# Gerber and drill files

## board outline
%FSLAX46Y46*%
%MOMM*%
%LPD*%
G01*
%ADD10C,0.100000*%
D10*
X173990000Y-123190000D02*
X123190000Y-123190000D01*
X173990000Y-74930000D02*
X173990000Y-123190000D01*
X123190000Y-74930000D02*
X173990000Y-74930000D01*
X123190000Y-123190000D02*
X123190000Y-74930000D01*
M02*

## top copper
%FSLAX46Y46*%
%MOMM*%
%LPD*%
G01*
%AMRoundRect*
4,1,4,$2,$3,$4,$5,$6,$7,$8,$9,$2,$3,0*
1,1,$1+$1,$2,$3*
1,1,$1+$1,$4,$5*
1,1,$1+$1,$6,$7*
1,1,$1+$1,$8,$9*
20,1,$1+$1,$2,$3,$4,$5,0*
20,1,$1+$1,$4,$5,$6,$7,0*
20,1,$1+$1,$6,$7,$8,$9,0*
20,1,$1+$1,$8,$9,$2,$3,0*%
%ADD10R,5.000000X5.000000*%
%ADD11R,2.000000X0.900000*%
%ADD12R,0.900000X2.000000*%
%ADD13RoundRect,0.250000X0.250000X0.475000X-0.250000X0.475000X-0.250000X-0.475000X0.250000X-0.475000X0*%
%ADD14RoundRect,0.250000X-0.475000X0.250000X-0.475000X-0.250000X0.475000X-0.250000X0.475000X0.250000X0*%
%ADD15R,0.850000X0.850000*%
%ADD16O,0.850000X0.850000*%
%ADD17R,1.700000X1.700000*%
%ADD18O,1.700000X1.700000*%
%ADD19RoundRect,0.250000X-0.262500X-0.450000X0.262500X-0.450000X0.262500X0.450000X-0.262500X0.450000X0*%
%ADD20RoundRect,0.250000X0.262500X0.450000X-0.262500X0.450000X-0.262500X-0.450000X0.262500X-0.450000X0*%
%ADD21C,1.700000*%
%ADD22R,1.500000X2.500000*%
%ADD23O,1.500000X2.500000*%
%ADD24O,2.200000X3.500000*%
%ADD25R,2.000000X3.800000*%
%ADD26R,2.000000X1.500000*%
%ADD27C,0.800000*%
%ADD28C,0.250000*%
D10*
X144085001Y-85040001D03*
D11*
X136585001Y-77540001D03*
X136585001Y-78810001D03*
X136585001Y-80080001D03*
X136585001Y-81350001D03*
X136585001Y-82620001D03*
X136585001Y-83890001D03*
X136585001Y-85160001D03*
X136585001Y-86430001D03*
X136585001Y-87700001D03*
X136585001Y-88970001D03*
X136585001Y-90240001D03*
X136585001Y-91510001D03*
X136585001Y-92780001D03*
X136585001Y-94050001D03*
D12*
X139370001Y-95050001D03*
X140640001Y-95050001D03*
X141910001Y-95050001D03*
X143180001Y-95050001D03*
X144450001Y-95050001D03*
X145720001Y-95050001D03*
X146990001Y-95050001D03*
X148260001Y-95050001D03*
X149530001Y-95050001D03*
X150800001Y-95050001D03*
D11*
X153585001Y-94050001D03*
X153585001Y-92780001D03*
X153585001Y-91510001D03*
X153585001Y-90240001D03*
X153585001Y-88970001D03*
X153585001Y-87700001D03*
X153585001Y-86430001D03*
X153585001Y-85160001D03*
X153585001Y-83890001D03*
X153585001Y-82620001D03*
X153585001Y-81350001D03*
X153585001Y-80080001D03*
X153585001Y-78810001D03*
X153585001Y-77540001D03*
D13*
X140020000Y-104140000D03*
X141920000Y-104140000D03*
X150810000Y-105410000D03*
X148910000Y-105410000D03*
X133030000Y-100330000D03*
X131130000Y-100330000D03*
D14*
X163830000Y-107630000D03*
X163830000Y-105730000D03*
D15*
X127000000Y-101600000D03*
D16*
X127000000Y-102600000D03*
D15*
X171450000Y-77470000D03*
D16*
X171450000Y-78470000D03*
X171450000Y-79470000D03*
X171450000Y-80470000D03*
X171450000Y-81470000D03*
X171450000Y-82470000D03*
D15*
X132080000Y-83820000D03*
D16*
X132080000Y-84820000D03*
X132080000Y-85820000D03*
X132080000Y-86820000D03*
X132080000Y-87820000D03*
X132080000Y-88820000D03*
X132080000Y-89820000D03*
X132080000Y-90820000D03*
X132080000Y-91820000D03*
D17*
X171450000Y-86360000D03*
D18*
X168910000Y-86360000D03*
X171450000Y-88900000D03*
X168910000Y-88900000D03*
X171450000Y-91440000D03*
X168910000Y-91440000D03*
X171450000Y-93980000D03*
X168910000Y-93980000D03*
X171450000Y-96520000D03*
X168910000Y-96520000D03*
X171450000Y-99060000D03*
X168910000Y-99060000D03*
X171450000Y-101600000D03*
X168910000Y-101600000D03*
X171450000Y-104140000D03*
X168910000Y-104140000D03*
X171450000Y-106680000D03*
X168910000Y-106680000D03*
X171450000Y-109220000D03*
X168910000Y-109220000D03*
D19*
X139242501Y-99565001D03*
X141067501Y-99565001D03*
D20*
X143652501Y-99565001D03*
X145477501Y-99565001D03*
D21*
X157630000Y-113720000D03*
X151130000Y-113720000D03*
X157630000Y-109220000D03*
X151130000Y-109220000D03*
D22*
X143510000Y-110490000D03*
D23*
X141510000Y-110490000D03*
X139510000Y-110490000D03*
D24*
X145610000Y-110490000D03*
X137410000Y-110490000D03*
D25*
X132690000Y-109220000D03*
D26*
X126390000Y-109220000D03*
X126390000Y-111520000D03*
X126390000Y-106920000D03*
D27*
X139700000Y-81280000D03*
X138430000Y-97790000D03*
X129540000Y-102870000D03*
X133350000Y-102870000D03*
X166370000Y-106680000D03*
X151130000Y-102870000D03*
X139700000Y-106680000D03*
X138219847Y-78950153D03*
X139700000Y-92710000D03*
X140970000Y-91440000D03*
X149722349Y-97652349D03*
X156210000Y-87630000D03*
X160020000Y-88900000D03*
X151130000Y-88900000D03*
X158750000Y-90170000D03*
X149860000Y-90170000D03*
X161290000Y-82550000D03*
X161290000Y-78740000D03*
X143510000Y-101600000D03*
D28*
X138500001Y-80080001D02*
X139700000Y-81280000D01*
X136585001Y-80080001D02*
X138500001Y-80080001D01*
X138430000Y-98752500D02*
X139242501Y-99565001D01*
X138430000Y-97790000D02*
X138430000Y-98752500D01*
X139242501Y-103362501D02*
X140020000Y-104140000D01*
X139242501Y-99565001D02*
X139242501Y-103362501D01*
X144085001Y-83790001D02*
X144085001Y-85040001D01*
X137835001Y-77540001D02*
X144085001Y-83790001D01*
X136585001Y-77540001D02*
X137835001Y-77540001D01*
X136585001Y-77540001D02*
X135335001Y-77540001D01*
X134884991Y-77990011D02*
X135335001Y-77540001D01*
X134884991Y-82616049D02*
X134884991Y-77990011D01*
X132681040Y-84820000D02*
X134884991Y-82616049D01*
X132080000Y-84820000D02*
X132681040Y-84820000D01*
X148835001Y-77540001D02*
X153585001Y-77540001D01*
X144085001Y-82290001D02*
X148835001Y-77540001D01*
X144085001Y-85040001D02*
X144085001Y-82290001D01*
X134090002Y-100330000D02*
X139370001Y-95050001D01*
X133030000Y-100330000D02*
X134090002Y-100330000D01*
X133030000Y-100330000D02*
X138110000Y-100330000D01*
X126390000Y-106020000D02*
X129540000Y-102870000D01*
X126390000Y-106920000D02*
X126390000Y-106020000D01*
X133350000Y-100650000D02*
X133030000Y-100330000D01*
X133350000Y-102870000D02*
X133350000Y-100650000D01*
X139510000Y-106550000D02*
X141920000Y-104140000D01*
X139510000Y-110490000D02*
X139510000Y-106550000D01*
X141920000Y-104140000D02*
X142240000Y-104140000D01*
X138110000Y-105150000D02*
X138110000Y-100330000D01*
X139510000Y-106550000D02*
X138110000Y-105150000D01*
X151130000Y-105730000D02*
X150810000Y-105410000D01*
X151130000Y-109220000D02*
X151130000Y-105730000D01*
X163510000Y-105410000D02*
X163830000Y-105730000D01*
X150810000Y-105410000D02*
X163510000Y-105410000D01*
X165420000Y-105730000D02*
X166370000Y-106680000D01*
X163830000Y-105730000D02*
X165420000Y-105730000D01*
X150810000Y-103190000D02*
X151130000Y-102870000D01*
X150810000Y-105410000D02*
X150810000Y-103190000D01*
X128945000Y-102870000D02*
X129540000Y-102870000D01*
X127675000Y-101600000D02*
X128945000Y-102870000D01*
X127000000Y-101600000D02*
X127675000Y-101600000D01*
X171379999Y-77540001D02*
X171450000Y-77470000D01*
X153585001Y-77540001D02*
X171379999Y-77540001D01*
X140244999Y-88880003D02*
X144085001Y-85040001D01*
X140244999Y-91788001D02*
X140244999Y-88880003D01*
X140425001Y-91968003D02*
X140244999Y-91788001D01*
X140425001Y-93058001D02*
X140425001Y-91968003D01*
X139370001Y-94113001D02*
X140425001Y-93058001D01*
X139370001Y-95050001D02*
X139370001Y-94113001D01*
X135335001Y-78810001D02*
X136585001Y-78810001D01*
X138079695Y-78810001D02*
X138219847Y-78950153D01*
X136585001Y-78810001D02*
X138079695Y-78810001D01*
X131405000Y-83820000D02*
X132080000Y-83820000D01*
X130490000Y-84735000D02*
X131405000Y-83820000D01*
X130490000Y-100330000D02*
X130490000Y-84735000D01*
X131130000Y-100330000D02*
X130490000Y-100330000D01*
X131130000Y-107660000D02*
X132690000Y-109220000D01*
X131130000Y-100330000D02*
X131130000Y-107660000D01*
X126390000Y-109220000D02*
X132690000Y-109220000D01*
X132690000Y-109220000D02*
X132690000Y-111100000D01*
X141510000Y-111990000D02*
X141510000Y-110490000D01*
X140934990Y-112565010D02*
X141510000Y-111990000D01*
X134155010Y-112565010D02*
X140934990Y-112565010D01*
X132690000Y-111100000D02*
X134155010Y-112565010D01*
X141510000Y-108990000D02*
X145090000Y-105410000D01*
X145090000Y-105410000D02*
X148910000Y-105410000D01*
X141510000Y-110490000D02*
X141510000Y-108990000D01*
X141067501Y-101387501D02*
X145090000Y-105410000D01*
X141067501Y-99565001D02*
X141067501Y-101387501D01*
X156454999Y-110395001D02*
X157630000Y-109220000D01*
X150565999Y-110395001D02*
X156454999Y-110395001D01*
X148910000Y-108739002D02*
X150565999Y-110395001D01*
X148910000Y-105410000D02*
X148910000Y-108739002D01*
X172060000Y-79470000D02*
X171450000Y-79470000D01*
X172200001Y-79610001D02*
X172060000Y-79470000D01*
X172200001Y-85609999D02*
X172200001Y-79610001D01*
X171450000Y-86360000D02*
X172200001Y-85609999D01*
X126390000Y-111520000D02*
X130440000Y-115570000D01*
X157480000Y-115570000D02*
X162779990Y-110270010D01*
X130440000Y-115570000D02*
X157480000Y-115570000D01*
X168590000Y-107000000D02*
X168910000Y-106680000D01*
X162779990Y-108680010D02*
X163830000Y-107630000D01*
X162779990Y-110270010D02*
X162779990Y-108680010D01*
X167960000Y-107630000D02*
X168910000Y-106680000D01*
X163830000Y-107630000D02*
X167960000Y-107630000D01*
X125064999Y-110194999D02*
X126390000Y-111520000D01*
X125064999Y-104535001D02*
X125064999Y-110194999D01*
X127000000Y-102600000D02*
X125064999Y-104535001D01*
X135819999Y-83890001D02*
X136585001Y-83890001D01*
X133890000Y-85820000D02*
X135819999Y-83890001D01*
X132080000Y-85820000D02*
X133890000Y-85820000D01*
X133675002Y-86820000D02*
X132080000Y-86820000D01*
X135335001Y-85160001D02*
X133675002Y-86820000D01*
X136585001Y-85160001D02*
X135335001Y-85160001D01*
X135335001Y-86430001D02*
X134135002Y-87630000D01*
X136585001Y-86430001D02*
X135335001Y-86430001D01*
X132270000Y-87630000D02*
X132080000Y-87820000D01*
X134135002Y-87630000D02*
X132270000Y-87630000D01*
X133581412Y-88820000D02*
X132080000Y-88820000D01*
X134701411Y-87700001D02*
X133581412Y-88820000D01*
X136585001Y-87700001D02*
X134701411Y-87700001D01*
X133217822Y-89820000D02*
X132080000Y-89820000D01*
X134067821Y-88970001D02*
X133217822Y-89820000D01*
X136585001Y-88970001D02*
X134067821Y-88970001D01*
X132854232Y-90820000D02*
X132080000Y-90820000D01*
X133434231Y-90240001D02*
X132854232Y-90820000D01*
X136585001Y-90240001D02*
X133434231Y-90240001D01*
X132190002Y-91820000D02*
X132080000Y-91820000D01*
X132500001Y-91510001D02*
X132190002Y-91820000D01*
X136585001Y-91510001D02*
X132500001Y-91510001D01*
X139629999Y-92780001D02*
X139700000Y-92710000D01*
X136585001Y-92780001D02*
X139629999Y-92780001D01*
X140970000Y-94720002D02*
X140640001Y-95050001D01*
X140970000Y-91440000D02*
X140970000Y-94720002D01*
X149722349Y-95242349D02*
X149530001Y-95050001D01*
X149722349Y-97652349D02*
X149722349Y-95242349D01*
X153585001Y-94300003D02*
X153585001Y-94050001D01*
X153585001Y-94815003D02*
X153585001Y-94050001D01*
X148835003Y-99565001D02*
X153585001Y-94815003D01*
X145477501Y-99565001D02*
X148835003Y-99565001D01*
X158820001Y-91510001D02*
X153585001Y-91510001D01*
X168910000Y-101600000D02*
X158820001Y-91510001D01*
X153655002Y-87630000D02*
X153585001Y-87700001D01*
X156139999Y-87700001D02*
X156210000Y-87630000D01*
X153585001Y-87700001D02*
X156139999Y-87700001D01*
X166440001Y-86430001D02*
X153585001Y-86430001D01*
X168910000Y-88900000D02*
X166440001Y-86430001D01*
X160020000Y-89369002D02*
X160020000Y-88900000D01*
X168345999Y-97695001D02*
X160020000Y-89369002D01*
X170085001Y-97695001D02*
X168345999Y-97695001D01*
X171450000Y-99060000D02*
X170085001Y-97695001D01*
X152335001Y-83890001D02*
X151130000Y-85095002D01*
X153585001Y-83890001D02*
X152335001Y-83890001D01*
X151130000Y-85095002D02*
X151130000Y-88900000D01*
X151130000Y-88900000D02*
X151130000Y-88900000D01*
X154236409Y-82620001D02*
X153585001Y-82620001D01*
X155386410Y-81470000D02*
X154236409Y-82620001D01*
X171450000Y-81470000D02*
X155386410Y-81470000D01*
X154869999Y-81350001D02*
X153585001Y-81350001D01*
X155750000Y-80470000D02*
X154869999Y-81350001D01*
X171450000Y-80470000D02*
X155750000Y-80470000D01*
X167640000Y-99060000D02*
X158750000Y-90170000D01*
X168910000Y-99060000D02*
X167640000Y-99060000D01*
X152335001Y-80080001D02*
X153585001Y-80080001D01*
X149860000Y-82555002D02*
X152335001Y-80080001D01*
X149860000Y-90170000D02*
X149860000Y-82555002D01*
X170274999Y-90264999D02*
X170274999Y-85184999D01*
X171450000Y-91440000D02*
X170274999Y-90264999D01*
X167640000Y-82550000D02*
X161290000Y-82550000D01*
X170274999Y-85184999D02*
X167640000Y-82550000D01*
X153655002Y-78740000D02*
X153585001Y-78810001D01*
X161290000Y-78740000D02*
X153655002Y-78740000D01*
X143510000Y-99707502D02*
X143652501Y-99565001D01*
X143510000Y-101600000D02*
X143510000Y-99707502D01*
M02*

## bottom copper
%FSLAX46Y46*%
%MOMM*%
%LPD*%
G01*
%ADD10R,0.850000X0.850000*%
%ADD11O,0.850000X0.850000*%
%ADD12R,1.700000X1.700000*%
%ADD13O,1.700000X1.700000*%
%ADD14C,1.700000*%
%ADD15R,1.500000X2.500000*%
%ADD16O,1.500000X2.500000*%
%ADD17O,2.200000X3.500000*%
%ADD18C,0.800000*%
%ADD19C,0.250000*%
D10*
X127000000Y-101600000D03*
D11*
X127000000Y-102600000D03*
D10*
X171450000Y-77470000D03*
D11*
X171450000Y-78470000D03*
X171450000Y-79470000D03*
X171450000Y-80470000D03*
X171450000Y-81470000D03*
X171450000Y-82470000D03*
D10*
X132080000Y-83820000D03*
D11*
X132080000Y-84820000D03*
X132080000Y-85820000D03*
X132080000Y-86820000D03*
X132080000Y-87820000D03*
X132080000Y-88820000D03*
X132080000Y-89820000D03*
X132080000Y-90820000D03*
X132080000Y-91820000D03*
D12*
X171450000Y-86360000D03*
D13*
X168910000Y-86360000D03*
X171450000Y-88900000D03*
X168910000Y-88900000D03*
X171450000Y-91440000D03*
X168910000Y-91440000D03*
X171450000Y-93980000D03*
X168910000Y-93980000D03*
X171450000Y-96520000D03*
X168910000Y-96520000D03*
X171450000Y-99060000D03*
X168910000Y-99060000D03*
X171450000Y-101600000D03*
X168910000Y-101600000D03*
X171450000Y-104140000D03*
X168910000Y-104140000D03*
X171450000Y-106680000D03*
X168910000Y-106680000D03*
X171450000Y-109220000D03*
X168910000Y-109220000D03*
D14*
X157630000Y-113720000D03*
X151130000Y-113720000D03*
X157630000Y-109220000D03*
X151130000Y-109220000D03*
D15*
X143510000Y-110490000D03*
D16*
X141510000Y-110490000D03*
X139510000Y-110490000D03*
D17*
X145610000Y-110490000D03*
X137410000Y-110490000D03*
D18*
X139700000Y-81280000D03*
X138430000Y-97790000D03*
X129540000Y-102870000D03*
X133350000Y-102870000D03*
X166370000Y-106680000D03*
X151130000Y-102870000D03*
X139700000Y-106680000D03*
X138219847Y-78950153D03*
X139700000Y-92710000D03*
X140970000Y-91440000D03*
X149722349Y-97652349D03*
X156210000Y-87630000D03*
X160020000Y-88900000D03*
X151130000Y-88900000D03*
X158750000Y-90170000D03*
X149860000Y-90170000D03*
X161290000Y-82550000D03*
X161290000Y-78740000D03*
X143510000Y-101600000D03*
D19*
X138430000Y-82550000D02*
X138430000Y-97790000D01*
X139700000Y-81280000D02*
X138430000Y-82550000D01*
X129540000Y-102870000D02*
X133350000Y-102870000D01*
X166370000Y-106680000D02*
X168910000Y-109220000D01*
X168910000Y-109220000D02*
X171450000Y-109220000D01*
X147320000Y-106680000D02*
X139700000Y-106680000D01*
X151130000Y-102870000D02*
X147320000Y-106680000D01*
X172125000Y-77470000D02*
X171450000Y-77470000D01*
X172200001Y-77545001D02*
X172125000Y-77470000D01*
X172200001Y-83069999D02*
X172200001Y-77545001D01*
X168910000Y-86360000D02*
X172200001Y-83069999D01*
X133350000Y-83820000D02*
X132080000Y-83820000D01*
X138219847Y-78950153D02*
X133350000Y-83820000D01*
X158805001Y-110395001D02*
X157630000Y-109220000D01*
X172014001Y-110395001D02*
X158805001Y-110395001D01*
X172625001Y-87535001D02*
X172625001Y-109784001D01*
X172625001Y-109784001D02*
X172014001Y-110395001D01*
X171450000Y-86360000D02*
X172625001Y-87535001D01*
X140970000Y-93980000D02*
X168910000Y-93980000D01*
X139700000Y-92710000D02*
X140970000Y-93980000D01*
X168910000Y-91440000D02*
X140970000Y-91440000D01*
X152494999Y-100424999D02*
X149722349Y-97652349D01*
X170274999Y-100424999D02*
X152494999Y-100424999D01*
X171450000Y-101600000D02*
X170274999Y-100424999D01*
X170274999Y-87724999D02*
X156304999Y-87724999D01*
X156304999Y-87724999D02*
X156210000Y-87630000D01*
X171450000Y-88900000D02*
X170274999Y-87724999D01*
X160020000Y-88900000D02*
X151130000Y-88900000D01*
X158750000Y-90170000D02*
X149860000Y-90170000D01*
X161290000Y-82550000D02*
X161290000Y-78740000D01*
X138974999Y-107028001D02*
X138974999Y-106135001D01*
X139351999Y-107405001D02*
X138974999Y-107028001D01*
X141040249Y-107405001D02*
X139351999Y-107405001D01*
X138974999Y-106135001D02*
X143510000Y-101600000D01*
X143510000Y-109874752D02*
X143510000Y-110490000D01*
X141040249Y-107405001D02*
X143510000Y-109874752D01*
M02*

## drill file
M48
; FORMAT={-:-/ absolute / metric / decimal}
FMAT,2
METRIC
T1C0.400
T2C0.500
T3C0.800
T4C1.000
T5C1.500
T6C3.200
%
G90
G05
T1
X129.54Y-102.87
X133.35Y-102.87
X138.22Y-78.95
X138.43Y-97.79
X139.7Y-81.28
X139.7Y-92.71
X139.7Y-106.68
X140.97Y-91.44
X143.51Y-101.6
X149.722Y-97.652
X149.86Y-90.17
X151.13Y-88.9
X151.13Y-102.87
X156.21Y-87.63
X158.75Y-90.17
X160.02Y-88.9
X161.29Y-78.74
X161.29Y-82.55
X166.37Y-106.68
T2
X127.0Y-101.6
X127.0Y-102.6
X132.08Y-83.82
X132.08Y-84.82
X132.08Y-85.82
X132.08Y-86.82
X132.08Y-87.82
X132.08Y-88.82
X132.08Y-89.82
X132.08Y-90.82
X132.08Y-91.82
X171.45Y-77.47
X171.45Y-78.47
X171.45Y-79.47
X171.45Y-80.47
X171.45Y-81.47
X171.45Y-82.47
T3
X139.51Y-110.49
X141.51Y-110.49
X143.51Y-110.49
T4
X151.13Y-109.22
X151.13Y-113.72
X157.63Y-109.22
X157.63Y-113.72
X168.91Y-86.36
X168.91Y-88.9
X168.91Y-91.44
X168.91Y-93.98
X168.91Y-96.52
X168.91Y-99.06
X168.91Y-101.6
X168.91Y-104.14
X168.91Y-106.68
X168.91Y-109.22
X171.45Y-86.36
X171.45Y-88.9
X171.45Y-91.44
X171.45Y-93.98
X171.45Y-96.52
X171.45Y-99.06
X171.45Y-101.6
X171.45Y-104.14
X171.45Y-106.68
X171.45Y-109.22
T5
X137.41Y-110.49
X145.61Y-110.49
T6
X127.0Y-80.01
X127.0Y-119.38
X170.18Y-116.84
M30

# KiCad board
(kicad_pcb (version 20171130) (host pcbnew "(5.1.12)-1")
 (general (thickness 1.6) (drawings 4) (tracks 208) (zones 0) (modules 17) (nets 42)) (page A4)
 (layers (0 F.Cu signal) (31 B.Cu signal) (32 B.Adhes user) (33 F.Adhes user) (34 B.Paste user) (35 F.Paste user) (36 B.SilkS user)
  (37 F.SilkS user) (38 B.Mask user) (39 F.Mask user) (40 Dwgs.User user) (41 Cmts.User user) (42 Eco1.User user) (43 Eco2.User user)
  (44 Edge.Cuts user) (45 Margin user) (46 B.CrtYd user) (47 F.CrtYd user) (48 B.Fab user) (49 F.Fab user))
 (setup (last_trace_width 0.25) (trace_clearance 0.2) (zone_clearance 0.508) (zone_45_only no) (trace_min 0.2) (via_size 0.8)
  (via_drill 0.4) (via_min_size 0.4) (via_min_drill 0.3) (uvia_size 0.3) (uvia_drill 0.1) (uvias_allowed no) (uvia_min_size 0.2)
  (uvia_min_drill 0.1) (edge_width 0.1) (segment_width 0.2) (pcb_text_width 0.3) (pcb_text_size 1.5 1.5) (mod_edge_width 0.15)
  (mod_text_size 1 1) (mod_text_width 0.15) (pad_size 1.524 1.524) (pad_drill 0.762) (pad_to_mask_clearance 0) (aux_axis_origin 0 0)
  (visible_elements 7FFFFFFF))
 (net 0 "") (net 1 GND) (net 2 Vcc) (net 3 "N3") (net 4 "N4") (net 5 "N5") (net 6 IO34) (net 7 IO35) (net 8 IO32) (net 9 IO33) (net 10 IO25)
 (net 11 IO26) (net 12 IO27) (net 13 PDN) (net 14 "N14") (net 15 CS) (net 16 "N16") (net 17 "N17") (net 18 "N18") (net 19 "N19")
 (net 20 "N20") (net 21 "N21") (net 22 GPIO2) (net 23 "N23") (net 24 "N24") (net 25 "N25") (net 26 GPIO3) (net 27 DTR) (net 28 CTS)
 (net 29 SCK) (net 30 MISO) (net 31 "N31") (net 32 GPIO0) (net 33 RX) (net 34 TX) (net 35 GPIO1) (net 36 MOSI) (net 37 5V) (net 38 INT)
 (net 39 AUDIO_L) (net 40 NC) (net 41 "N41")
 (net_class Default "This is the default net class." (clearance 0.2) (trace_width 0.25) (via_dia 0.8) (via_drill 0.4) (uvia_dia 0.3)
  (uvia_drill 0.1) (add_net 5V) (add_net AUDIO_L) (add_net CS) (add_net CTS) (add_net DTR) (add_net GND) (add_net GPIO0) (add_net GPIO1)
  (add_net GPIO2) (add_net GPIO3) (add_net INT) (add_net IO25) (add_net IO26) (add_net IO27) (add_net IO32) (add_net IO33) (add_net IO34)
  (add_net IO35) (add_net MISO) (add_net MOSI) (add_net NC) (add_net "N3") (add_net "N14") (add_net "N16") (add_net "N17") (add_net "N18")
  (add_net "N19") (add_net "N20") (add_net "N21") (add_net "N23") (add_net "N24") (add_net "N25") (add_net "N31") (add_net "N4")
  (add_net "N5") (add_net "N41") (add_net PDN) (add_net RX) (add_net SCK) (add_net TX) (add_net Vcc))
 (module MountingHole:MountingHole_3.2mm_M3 (layer F.Cu) (at 127 119.38)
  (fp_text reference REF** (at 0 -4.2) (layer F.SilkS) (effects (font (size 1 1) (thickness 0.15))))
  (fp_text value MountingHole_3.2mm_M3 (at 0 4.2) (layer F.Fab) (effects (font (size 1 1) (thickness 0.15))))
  (pad 1 np_thru_hole circle (at 0 0) (size 3.2 3.2) (drill 3.2) (layers *.Cu *.Mask)))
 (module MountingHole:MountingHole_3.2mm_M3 (layer F.Cu) (at 170.18 116.84)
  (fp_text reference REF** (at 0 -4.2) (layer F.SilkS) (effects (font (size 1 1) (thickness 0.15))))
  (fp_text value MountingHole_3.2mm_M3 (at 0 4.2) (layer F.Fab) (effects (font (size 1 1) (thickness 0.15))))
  (pad 1 np_thru_hole circle (at 0 0) (size 3.2 3.2) (drill 3.2) (layers *.Cu *.Mask)))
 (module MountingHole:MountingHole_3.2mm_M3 (layer F.Cu) (at 127 80.01)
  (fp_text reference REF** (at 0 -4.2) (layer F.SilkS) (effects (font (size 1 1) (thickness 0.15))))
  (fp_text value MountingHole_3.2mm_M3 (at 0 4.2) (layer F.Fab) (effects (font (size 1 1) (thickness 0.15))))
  (pad 1 np_thru_hole circle (at 0 0) (size 3.2 3.2) (drill 3.2) (layers *.Cu *.Mask)))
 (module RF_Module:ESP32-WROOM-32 (layer F.Cu) (at 145.085001 85.795001)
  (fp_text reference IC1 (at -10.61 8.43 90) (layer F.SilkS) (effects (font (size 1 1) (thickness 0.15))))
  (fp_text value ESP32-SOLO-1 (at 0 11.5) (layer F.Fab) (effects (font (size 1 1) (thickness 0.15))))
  (pad 39 smd rect (at -1 -0.755) (size 5 5) (layers F.Cu F.Paste F.Mask) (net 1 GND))
  (pad 1 smd rect (at -8.5 -8.255) (size 2 0.9) (layers F.Cu F.Paste F.Mask) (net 1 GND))
  (pad 2 smd rect (at -8.5 -6.985) (size 2 0.9) (layers F.Cu F.Paste F.Mask) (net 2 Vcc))
  (pad 3 smd rect (at -8.5 -5.715) (size 2 0.9) (layers F.Cu F.Paste F.Mask) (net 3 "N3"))
  (pad 4 smd rect (at -8.5 -4.445) (size 2 0.9) (layers F.Cu F.Paste F.Mask) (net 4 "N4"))
  (pad 5 smd rect (at -8.5 -3.175) (size 2 0.9) (layers F.Cu F.Paste F.Mask) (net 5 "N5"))
  (pad 6 smd rect (at -8.5 -1.905) (size 2 0.9) (layers F.Cu F.Paste F.Mask) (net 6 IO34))
  (pad 7 smd rect (at -8.5 -0.635) (size 2 0.9) (layers F.Cu F.Paste F.Mask) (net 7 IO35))
  (pad 8 smd rect (at -8.5 0.635) (size 2 0.9) (layers F.Cu F.Paste F.Mask) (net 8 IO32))
  (pad 9 smd rect (at -8.5 1.905) (size 2 0.9) (layers F.Cu F.Paste F.Mask) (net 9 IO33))
  (pad 10 smd rect (at -8.5 3.175) (size 2 0.9) (layers F.Cu F.Paste F.Mask) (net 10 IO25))
  (pad 11 smd rect (at -8.5 4.445) (size 2 0.9) (layers F.Cu F.Paste F.Mask) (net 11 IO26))
  (pad 12 smd rect (at -8.5 5.715) (size 2 0.9) (layers F.Cu F.Paste F.Mask) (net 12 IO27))
  (pad 13 smd rect (at -8.5 6.985) (size 2 0.9) (layers F.Cu F.Paste F.Mask) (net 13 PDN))
  (pad 14 smd rect (at -8.5 8.255) (size 2 0.9) (layers F.Cu F.Paste F.Mask) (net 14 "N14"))
  (pad 15 smd rect (at -5.715 9.255 90) (size 2 0.9) (layers F.Cu F.Paste F.Mask) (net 1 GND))
  (pad 16 smd rect (at -4.445 9.255 90) (size 2 0.9) (layers F.Cu F.Paste F.Mask) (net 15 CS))
  (pad 17 smd rect (at -3.175 9.255 90) (size 2 0.9) (layers F.Cu F.Paste F.Mask) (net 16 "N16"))
  (pad 18 smd rect (at -1.905 9.255 90) (size 2 0.9) (layers F.Cu F.Paste F.Mask) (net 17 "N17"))
  (pad 19 smd rect (at -0.635 9.255 90) (size 2 0.9) (layers F.Cu F.Paste F.Mask) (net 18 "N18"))
  (pad 20 smd rect (at 0.635 9.255 90) (size 2 0.9) (layers F.Cu F.Paste F.Mask) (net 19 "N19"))
  (pad 21 smd rect (at 1.905 9.255 90) (size 2 0.9) (layers F.Cu F.Paste F.Mask) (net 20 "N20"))
  (pad 22 smd rect (at 3.175 9.255 90) (size 2 0.9) (layers F.Cu F.Paste F.Mask) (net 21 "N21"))
  (pad 23 smd rect (at 4.445 9.255 90) (size 2 0.9) (layers F.Cu F.Paste F.Mask) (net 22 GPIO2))
  (pad 24 smd rect (at 5.715 9.255 90) (size 2 0.9) (layers F.Cu F.Paste F.Mask) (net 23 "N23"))
  (pad 25 smd rect (at 8.5 8.255) (size 2 0.9) (layers F.Cu F.Paste F.Mask) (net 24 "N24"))
  (pad 26 smd rect (at 8.5 6.985) (size 2 0.9) (layers F.Cu F.Paste F.Mask) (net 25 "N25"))
  (pad 27 smd rect (at 8.5 5.715) (size 2 0.9) (layers F.Cu F.Paste F.Mask) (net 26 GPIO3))
  (pad 28 smd rect (at 8.5 4.445) (size 2 0.9) (layers F.Cu F.Paste F.Mask) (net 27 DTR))
  (pad 29 smd rect (at 8.5 3.175) (size 2 0.9) (layers F.Cu F.Paste F.Mask) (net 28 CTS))
  (pad 30 smd rect (at 8.5 1.905) (size 2 0.9) (layers F.Cu F.Paste F.Mask) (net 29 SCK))
  (pad 31 smd rect (at 8.5 0.635) (size 2 0.9) (layers F.Cu F.Paste F.Mask) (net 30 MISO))
  (pad 32 smd rect (at 8.5 -0.635) (size 2 0.9) (layers F.Cu F.Paste F.Mask) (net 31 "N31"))
  (pad 33 smd rect (at 8.5 -1.905) (size 2 0.9) (layers F.Cu F.Paste F.Mask) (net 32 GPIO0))
  (pad 34 smd rect (at 8.5 -3.175) (size 2 0.9) (layers F.Cu F.Paste F.Mask) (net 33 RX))
  (pad 35 smd rect (at 8.5 -4.445) (size 2 0.9) (layers F.Cu F.Paste F.Mask) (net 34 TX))
  (pad 36 smd rect (at 8.5 -5.715) (size 2 0.9) (layers F.Cu F.Paste F.Mask) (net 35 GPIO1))
  (pad 37 smd rect (at 8.5 -6.985) (size 2 0.9) (layers F.Cu F.Paste F.Mask) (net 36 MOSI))
  (pad 38 smd rect (at 8.5 -8.255) (size 2 0.9) (layers F.Cu F.Paste F.Mask) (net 1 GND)))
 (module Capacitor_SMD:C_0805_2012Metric (layer F.Cu) (at 140.97 104.14 180)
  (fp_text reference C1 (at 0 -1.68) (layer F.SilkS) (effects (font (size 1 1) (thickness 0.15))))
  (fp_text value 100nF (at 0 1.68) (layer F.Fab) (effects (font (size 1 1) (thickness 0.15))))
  (pad 2 smd roundrect (at 0.95 0 180) (size 1 1.45) (layers F.Cu F.Paste F.Mask) (roundrect_rratio 0.25) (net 3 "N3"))
  (pad 1 smd roundrect (at -0.95 0 180) (size 1 1.45) (layers F.Cu F.Paste F.Mask) (roundrect_rratio 0.25) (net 1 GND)))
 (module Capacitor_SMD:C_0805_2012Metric (layer F.Cu) (at 149.86 105.41 180)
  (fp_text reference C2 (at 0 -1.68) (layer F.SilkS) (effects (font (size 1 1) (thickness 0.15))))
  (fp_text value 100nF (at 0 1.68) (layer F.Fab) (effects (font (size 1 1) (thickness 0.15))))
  (pad 1 smd roundrect (at -0.95 0 180) (size 1 1.45) (layers F.Cu F.Paste F.Mask) (roundrect_rratio 0.25) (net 1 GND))
  (pad 2 smd roundrect (at 0.95 0 180) (size 1 1.45) (layers F.Cu F.Paste F.Mask) (roundrect_rratio 0.25) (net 2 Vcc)))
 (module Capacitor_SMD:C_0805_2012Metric (layer F.Cu) (at 132.08 100.33 180)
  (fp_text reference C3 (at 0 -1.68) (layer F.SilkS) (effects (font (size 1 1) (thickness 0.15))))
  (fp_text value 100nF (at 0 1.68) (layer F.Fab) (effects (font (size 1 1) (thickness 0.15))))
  (pad 1 smd roundrect (at -0.95 0 180) (size 1 1.45) (layers F.Cu F.Paste F.Mask) (roundrect_rratio 0.25) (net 1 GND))
  (pad 2 smd roundrect (at 0.95 0 180) (size 1 1.45) (layers F.Cu F.Paste F.Mask) (roundrect_rratio 0.25) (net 2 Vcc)))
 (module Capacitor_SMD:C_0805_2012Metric (layer F.Cu) (at 163.83 106.68 270)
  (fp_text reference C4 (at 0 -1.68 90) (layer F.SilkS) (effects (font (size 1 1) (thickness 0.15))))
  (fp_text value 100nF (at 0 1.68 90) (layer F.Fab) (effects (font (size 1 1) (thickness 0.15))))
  (pad 2 smd roundrect (at 0.95 0 270) (size 1 1.45) (layers F.Cu F.Paste F.Mask) (roundrect_rratio 0.25) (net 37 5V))
  (pad 1 smd roundrect (at -0.95 0 270) (size 1 1.45) (layers F.Cu F.Paste F.Mask) (roundrect_rratio 0.25) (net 1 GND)))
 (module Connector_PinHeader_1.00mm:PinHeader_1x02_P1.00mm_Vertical (layer F.Cu) (at 127 101.6)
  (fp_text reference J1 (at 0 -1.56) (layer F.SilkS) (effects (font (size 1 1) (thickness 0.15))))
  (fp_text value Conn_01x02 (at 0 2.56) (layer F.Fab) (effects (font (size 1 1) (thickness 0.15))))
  (pad 1 thru_hole rect (at 0 0) (size 0.85 0.85) (drill 0.5) (layers *.Cu *.Mask) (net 1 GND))
  (pad 2 thru_hole oval (at 0 1) (size 0.85 0.85) (drill 0.5) (layers *.Cu *.Mask) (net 37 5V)))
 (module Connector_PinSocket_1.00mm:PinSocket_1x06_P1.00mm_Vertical (layer F.Cu) (at 171.45 77.47)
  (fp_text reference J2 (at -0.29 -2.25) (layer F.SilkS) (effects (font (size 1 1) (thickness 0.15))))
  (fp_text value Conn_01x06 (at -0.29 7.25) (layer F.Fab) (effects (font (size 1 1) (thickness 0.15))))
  (pad 1 thru_hole rect (at 0 0) (size 0.85 0.85) (drill 0.5) (layers *.Cu *.Mask) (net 1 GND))
  (pad 2 thru_hole oval (at 0 1) (size 0.85 0.85) (drill 0.5) (layers *.Cu *.Mask) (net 28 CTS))
  (pad 3 thru_hole oval (at 0 2) (size 0.85 0.85) (drill 0.5) (layers *.Cu *.Mask) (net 2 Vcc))
  (pad 4 thru_hole oval (at 0 3) (size 0.85 0.85) (drill 0.5) (layers *.Cu *.Mask) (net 34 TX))
  (pad 5 thru_hole oval (at 0 4) (size 0.85 0.85) (drill 0.5) (layers *.Cu *.Mask) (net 33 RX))
  (pad 6 thru_hole oval (at 0 5) (size 0.85 0.85) (drill 0.5) (layers *.Cu *.Mask) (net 27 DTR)))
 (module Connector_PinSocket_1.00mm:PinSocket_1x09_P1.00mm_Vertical (layer F.Cu) (at 132.08 83.82)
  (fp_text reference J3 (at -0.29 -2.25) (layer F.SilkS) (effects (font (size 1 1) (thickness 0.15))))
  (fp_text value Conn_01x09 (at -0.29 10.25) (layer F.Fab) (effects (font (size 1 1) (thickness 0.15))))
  (pad 1 thru_hole rect (at 0 0) (size 0.85 0.85) (drill 0.5) (layers *.Cu *.Mask) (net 2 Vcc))
  (pad 2 thru_hole oval (at 0 1) (size 0.85 0.85) (drill 0.5) (layers *.Cu *.Mask) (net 1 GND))
  (pad 3 thru_hole oval (at 0 2) (size 0.85 0.85) (drill 0.5) (layers *.Cu *.Mask) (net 6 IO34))
  (pad 4 thru_hole oval (at 0 3) (size 0.85 0.85) (drill 0.5) (layers *.Cu *.Mask) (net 7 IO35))
  (pad 5 thru_hole oval (at 0 4) (size 0.85 0.85) (drill 0.5) (layers *.Cu *.Mask) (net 8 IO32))
  (pad 6 thru_hole oval (at 0 5) (size 0.85 0.85) (drill 0.5) (layers *.Cu *.Mask) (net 9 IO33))
  (pad 7 thru_hole oval (at 0 6) (size 0.85 0.85) (drill 0.5) (layers *.Cu *.Mask) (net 10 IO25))
  (pad 8 thru_hole oval (at 0 7) (size 0.85 0.85) (drill 0.5) (layers *.Cu *.Mask) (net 11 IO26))
  (pad 9 thru_hole oval (at 0 8) (size 0.85 0.85) (drill 0.5) (layers *.Cu *.Mask) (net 12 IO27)))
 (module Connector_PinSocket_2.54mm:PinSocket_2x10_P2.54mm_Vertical (layer F.Cu) (at 171.45 86.36)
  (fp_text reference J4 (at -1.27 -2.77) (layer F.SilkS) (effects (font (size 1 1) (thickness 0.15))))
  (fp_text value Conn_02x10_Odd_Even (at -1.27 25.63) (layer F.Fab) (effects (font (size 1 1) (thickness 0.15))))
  (pad 1 thru_hole rect (at 0 0) (size 1.7 1.7) (drill 1) (layers *.Cu *.Mask) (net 2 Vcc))
  (pad 2 thru_hole oval (at -2.54 0) (size 1.7 1.7) (drill 1) (layers *.Cu *.Mask) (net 1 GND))
  (pad 3 thru_hole oval (at 0 2.54) (size 1.7 1.7) (drill 1) (layers *.Cu *.Mask) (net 29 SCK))
  (pad 4 thru_hole oval (at -2.54 2.54) (size 1.7 1.7) (drill 1) (layers *.Cu *.Mask) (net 30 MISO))
  (pad 5 thru_hole oval (at 0 5.08) (size 1.7 1.7) (drill 1) (layers *.Cu *.Mask) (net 36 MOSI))
  (pad 6 thru_hole oval (at -2.54 5.08) (size 1.7 1.7) (drill 1) (layers *.Cu *.Mask) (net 15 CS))
  (pad 7 thru_hole oval (at 0 7.62) (size 1.7 1.7) (drill 1) (layers *.Cu *.Mask) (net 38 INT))
  (pad 8 thru_hole oval (at -2.54 7.62) (size 1.7 1.7) (drill 1) (layers *.Cu *.Mask) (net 13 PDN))
  (pad 9 thru_hole oval (at 0 10.16) (size 1.7 1.7) (drill 1) (layers *.Cu *.Mask) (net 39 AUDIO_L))
  (pad 10 thru_hole oval (at -2.54 10.16) (size 1.7 1.7) (drill 1) (layers *.Cu *.Mask) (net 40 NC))
  (pad 11 thru_hole oval (at 0 12.7) (size 1.7 1.7) (drill 1) (layers *.Cu *.Mask) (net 32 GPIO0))
  (pad 12 thru_hole oval (at -2.54 12.7) (size 1.7 1.7) (drill 1) (layers *.Cu *.Mask) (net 35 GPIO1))
  (pad 13 thru_hole oval (at 0 15.24) (size 1.7 1.7) (drill 1) (layers *.Cu *.Mask) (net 22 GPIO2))
  (pad 14 thru_hole oval (at -2.54 15.24) (size 1.7 1.7) (drill 1) (layers *.Cu *.Mask) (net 26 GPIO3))
  (pad 15 thru_hole oval (at 0 17.78) (size 1.7 1.7) (drill 1) (layers *.Cu *.Mask) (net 40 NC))
  (pad 16 thru_hole oval (at -2.54 17.78) (size 1.7 1.7) (drill 1) (layers *.Cu *.Mask) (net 40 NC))
  (pad 17 thru_hole oval (at 0 20.32) (size 1.7 1.7) (drill 1) (layers *.Cu *.Mask) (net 40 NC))
  (pad 18 thru_hole oval (at -2.54 20.32) (size 1.7 1.7) (drill 1) (layers *.Cu *.Mask) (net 37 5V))
  (pad 19 thru_hole oval (at 0 22.86) (size 1.7 1.7) (drill 1) (layers *.Cu *.Mask) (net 1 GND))
  (pad 20 thru_hole oval (at -2.54 22.86) (size 1.7 1.7) (drill 1) (layers *.Cu *.Mask) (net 1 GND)))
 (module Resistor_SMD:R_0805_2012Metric (layer F.Cu) (at 140.155001 99.565001)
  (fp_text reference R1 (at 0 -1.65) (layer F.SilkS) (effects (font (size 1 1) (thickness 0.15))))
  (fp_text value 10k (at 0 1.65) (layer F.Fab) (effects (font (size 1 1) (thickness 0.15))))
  (pad 1 smd roundrect (at -0.9125 0) (size 1.025 1.4) (layers F.Cu F.Paste F.Mask) (roundrect_rratio 0.243902) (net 3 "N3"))
  (pad 2 smd roundrect (at 0.9125 0) (size 1.025 1.4) (layers F.Cu F.Paste F.Mask) (roundrect_rratio 0.243902) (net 2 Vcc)))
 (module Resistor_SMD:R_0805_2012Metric (layer F.Cu) (at 144.565001 99.565001 180)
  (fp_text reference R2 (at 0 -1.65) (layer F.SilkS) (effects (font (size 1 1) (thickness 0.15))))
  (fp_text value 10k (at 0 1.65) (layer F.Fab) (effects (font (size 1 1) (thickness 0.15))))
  (pad 2 smd roundrect (at 0.9125 0 180) (size 1.025 1.4) (layers F.Cu F.Paste F.Mask) (roundrect_rratio 0.243902) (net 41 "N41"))
  (pad 1 smd roundrect (at -0.9125 0 180) (size 1.025 1.4) (layers F.Cu F.Paste F.Mask) (roundrect_rratio 0.243902) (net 24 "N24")))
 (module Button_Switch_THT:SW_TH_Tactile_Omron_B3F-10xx (layer F.Cu) (at 151.13 109.22)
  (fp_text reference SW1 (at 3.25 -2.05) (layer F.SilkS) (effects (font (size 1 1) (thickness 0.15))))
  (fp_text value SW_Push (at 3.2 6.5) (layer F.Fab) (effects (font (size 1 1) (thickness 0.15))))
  (pad 4 thru_hole circle (at 6.5 4.5) (size 1.7 1.7) (drill 1) (layers *.Cu *.Mask))
  (pad 3 thru_hole circle (at 0 4.5) (size 1.7 1.7) (drill 1) (layers *.Cu *.Mask))
  (pad 2 thru_hole circle (at 6.5 0) (size 1.7 1.7) (drill 1) (layers *.Cu *.Mask) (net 2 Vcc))
  (pad 1 thru_hole circle (at 0 0) (size 1.7 1.7) (drill 1) (layers *.Cu *.Mask) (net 1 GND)))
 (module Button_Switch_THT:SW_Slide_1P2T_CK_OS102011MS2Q (layer F.Cu) (at 143.51 110.49 180)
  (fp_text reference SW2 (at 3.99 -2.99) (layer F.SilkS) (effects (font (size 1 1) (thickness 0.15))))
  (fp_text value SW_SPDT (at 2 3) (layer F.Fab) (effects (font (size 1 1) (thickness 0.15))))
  (pad 1 thru_hole rect (at 0 0 180) (size 1.5 2.5) (drill 0.8) (layers *.Cu *.Mask) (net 41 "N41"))
  (pad 2 thru_hole oval (at 2 0 180) (size 1.5 2.5) (drill 0.8) (layers *.Cu *.Mask) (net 2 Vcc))
  (pad 3 thru_hole oval (at 4 0 180) (size 1.5 2.5) (drill 0.8) (layers *.Cu *.Mask) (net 1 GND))
  (pad "" thru_hole oval (at -2.1 0 180) (size 2.2 3.5) (drill 1.5) (layers *.Cu *.Mask))
  (pad "" thru_hole oval (at 6.1 0 180) (size 2.2 3.5) (drill 1.5) (layers *.Cu *.Mask)))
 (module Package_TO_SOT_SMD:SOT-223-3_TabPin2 (layer F.Cu) (at 129.54 109.22)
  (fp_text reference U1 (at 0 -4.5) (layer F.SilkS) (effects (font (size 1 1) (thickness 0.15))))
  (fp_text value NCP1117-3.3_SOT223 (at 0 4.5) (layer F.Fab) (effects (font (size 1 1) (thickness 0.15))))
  (pad 2 smd rect (at 3.15 0) (size 2 3.8) (layers F.Cu F.Paste F.Mask) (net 2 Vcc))
  (pad 2 smd rect (at -3.15 0) (size 2 1.5) (layers F.Cu F.Paste F.Mask) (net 2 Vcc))
  (pad 3 smd rect (at -3.15 2.3) (size 2 1.5) (layers F.Cu F.Paste F.Mask) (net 37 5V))
  (pad 1 smd rect (at -3.15 -2.3) (size 2 1.5) (layers F.Cu F.Paste F.Mask) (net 1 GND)))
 (gr_line (start 173.99 123.19) (end 123.19 123.19) (layer Edge.Cuts) (width 0.1))
 (gr_line (start 173.99 74.93) (end 173.99 123.19) (layer Edge.Cuts) (width 0.1))
 (gr_line (start 123.19 74.93) (end 173.99 74.93) (layer Edge.Cuts) (width 0.1))
 (gr_line (start 123.19 123.19) (end 123.19 74.93) (layer Edge.Cuts) (width 0.1))
 (via (at 139.7 81.28) (size 0.8) (drill 0.4) (layers F.Cu B.Cu) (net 3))
 (segment (start 138.500001 80.080001) (end 139.7 81.28) (width 0.25) (layer F.Cu) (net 3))
 (segment (start 136.585001 80.080001) (end 138.500001 80.080001) (width 0.25) (layer F.Cu) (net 3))
 (via (at 138.43 97.79) (size 0.8) (drill 0.4) (layers F.Cu B.Cu) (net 3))
 (segment (start 138.43 82.55) (end 138.43 97.79) (width 0.25) (layer B.Cu) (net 3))
 (segment (start 139.7 81.28) (end 138.43 82.55) (width 0.25) (layer B.Cu) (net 3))
 (segment (start 138.43 98.7525) (end 139.242501 99.565001) (width 0.25) (layer F.Cu) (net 3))
 (segment (start 138.43 97.79) (end 138.43 98.7525) (width 0.25) (layer F.Cu) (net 3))
 (segment (start 139.242501 103.362501) (end 140.02 104.14) (width 0.25) (layer F.Cu) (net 3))
 (segment (start 139.242501 99.565001) (end 139.242501 103.362501) (width 0.25) (layer F.Cu) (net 3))
 (segment (start 144.085001 83.790001) (end 144.085001 85.040001) (width 0.25) (layer F.Cu) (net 1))
 (segment (start 137.835001 77.540001) (end 144.085001 83.790001) (width 0.25) (layer F.Cu) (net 1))
 (segment (start 136.585001 77.540001) (end 137.835001 77.540001) (width 0.25) (layer F.Cu) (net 1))
 (segment (start 136.585001 77.540001) (end 135.335001 77.540001) (width 0.25) (layer F.Cu) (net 1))
 (segment (start 134.884991 77.990011) (end 135.335001 77.540001) (width 0.25) (layer F.Cu) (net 1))
 (segment (start 134.884991 82.616049) (end 134.884991 77.990011) (width 0.25) (layer F.Cu) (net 1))
 (segment (start 132.68104 84.82) (end 134.884991 82.616049) (width 0.25) (layer F.Cu) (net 1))
 (segment (start 132.08 84.82) (end 132.68104 84.82) (width 0.25) (layer F.Cu) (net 1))
 (segment (start 148.835001 77.540001) (end 153.585001 77.540001) (width 0.25) (layer F.Cu) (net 1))
 (segment (start 144.085001 82.290001) (end 148.835001 77.540001) (width 0.25) (layer F.Cu) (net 1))
 (segment (start 144.085001 85.040001) (end 144.085001 82.290001) (width 0.25) (layer F.Cu) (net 1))
 (segment (start 134.090002 100.33) (end 139.370001 95.050001) (width 0.25) (layer F.Cu) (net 1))
 (segment (start 133.03 100.33) (end 134.090002 100.33) (width 0.25) (layer F.Cu) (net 1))
 (segment (start 133.03 100.33) (end 138.11 100.33) (width 0.25) (layer F.Cu) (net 1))
 (via (at 129.54 102.87) (size 0.8) (drill 0.4) (layers F.Cu B.Cu) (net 1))
 (segment (start 126.39 106.02) (end 129.54 102.87) (width 0.25) (layer F.Cu) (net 1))
 (segment (start 126.39 106.92) (end 126.39 106.02) (width 0.25) (layer F.Cu) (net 1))
 (segment (start 129.54 102.87) (end 133.35 102.87) (width 0.25) (layer B.Cu) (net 1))
 (via (at 133.35 102.87) (size 0.8) (drill 0.4) (layers F.Cu B.Cu) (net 1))
 (segment (start 133.35 100.65) (end 133.03 100.33) (width 0.25) (layer F.Cu) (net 1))
 (segment (start 133.35 102.87) (end 133.35 100.65) (width 0.25) (layer F.Cu) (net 1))
 (segment (start 139.51 106.55) (end 141.92 104.14) (width 0.25) (layer F.Cu) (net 1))
 (segment (start 139.51 110.49) (end 139.51 106.55) (width 0.25) (layer F.Cu) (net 1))
 (segment (start 141.92 104.14) (end 142.24 104.14) (width 0.25) (layer F.Cu) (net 1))
 (segment (start 138.11 105.15) (end 138.11 100.33) (width 0.25) (layer F.Cu) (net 1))
 (segment (start 139.51 106.55) (end 138.11 105.15) (width 0.25) (layer F.Cu) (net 1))
 (segment (start 151.13 105.73) (end 150.81 105.41) (width 0.25) (layer F.Cu) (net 1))
 (segment (start 151.13 109.22) (end 151.13 105.73) (width 0.25) (layer F.Cu) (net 1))
 (segment (start 163.51 105.41) (end 163.83 105.73) (width 0.25) (layer F.Cu) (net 1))
 (segment (start 150.81 105.41) (end 163.51 105.41) (width 0.25) (layer F.Cu) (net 1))
 (via (at 166.37 106.68) (size 0.8) (drill 0.4) (layers F.Cu B.Cu) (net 1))
 (segment (start 165.42 105.73) (end 166.37 106.68) (width 0.25) (layer F.Cu) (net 1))
 (segment (start 163.83 105.73) (end 165.42 105.73) (width 0.25) (layer F.Cu) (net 1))
 (segment (start 166.37 106.68) (end 168.91 109.22) (width 0.25) (layer B.Cu) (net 1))
 (segment (start 168.91 109.22) (end 171.45 109.22) (width 0.25) (layer B.Cu) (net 1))
 (via (at 151.13 102.87) (size 0.8) (drill 0.4) (layers F.Cu B.Cu) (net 1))
 (segment (start 150.81 103.19) (end 151.13 102.87) (width 0.25) (layer F.Cu) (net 1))
 (segment (start 150.81 105.41) (end 150.81 103.19) (width 0.25) (layer F.Cu) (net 1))
 (via (at 139.7 106.68) (size 0.8) (drill 0.4) (layers F.Cu B.Cu) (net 1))
 (segment (start 147.32 106.68) (end 139.7 106.68) (width 0.25) (layer B.Cu) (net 1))
 (segment (start 151.13 102.87) (end 147.32 106.68) (width 0.25) (layer B.Cu) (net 1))
 (segment (start 128.945 102.87) (end 129.54 102.87) (width 0.25) (layer F.Cu) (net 1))
 (segment (start 127.675 101.6) (end 128.945 102.87) (width 0.25) (layer F.Cu) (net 1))
 (segment (start 127 101.6) (end 127.675 101.6) (width 0.25) (layer F.Cu) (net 1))
 (segment (start 171.379999 77.540001) (end 171.45 77.47) (width 0.25) (layer F.Cu) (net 1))
 (segment (start 153.585001 77.540001) (end 171.379999 77.540001) (width 0.25) (layer F.Cu) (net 1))
 (segment (start 172.125 77.47) (end 171.45 77.47) (width 0.25) (layer B.Cu) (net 1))
 (segment (start 172.200001 77.545001) (end 172.125 77.47) (width 0.25) (layer B.Cu) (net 1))
 (segment (start 172.200001 83.069999) (end 172.200001 77.545001) (width 0.25) (layer B.Cu) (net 1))
 (segment (start 168.91 86.36) (end 172.200001 83.069999) (width 0.25) (layer B.Cu) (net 1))
 (segment (start 140.244999 88.880003) (end 144.085001 85.040001) (width 0.25) (layer F.Cu) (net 1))
 (segment (start 140.244999 91.788001) (end 140.244999 88.880003) (width 0.25) (layer F.Cu) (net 1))
 (segment (start 140.425001 91.968003) (end 140.244999 91.788001) (width 0.25) (layer F.Cu) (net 1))
 (segment (start 140.425001 93.058001) (end 140.425001 91.968003) (width 0.25) (layer F.Cu) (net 1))
 (segment (start 139.370001 94.113001) (end 140.425001 93.058001) (width 0.25) (layer F.Cu) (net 1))
 (segment (start 139.370001 95.050001) (end 139.370001 94.113001) (width 0.25) (layer F.Cu) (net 1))
 (segment (start 135.335001 78.810001) (end 136.585001 78.810001) (width 0.25) (layer F.Cu) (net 2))
 (via (at 138.219847 78.950153) (size 0.8) (drill 0.4) (layers F.Cu B.Cu) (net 2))
 (segment (start 138.079695 78.810001) (end 138.219847 78.950153) (width 0.25) (layer F.Cu) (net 2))
 (segment (start 136.585001 78.810001) (end 138.079695 78.810001) (width 0.25) (layer F.Cu) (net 2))
 (segment (start 133.35 83.82) (end 132.08 83.82) (width 0.25) (layer B.Cu) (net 2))
 (segment (start 138.219847 78.950153) (end 133.35 83.82) (width 0.25) (layer B.Cu) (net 2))
 (segment (start 131.405 83.82) (end 132.08 83.82) (width 0.25) (layer F.Cu) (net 2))
 (segment (start 130.49 84.735) (end 131.405 83.82) (width 0.25) (layer F.Cu) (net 2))
 (segment (start 130.49 100.33) (end 130.49 84.735) (width 0.25) (layer F.Cu) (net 2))
 (segment (start 131.13 100.33) (end 130.49 100.33) (width 0.25) (layer F.Cu) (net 2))
 (segment (start 131.13 107.66) (end 132.69 109.22) (width 0.25) (layer F.Cu) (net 2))
 (segment (start 131.13 100.33) (end 131.13 107.66) (width 0.25) (layer F.Cu) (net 2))
 (segment (start 126.39 109.22) (end 132.69 109.22) (width 0.25) (layer F.Cu) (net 2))
 (segment (start 132.69 109.22) (end 132.69 111.1) (width 0.25) (layer F.Cu) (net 2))
 (segment (start 141.51 111.99) (end 141.51 110.49) (width 0.25) (layer F.Cu) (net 2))
 (segment (start 140.93499 112.56501) (end 141.51 111.99) (width 0.25) (layer F.Cu) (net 2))
 (segment (start 134.15501 112.56501) (end 140.93499 112.56501) (width 0.25) (layer F.Cu) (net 2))
 (segment (start 132.69 111.1) (end 134.15501 112.56501) (width 0.25) (layer F.Cu) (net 2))
 (segment (start 141.51 108.99) (end 145.09 105.41) (width 0.25) (layer F.Cu) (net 2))
 (segment (start 145.09 105.41) (end 148.91 105.41) (width 0.25) (layer F.Cu) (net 2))
 (segment (start 141.51 110.49) (end 141.51 108.99) (width 0.25) (layer F.Cu) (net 2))
 (segment (start 141.067501 101.387501) (end 145.09 105.41) (width 0.25) (layer F.Cu) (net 2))
 (segment (start 141.067501 99.565001) (end 141.067501 101.387501) (width 0.25) (layer F.Cu) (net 2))
 (segment (start 156.454999 110.395001) (end 157.63 109.22) (width 0.25) (layer F.Cu) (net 2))
 (segment (start 150.565999 110.395001) (end 156.454999 110.395001) (width 0.25) (layer F.Cu) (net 2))
 (segment (start 148.91 108.739002) (end 150.565999 110.395001) (width 0.25) (layer F.Cu) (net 2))
 (segment (start 148.91 105.41) (end 148.91 108.739002) (width 0.25) (layer F.Cu) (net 2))
 (segment (start 172.06 79.47) (end 171.45 79.47) (width 0.25) (layer F.Cu) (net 2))
 (segment (start 172.200001 79.610001) (end 172.06 79.47) (width 0.25) (layer F.Cu) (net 2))
 (segment (start 172.200001 85.609999) (end 172.200001 79.610001) (width 0.25) (layer F.Cu) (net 2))
 (segment (start 171.45 86.36) (end 172.200001 85.609999) (width 0.25) (layer F.Cu) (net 2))
 (segment (start 158.805001 110.395001) (end 157.63 109.22) (width 0.25) (layer B.Cu) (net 2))
 (segment (start 172.014001 110.395001) (end 158.805001 110.395001) (width 0.25) (layer B.Cu) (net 2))
 (segment (start 172.625001 87.535001) (end 172.625001 109.784001) (width 0.25) (layer B.Cu) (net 2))
 (segment (start 172.625001 109.784001) (end 172.014001 110.395001) (width 0.25) (layer B.Cu) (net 2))
 (segment (start 171.45 86.36) (end 172.625001 87.535001) (width 0.25) (layer B.Cu) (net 2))
 (segment (start 126.39 111.52) (end 130.44 115.57) (width 0.25) (layer F.Cu) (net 37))
 (segment (start 157.48 115.57) (end 162.77999 110.27001) (width 0.25) (layer F.Cu) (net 37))
 (segment (start 130.44 115.57) (end 157.48 115.57) (width 0.25) (layer F.Cu) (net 37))
 (segment (start 168.59 107) (end 168.91 106.68) (width 0.25) (layer F.Cu) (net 37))
 (segment (start 162.77999 108.68001) (end 163.83 107.63) (width 0.25) (layer F.Cu) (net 37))
 (segment (start 162.77999 110.27001) (end 162.77999 108.68001) (width 0.25) (layer F.Cu) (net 37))
 (segment (start 167.96 107.63) (end 168.91 106.68) (width 0.25) (layer F.Cu) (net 37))
 (segment (start 163.83 107.63) (end 167.96 107.63) (width 0.25) (layer F.Cu) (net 37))
 (segment (start 125.064999 110.194999) (end 126.39 111.52) (width 0.25) (layer F.Cu) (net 37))
 (segment (start 125.064999 104.535001) (end 125.064999 110.194999) (width 0.25) (layer F.Cu) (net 37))
 (segment (start 127 102.6) (end 125.064999 104.535001) (width 0.25) (layer F.Cu) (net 37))
 (segment (start 135.819999 83.890001) (end 136.585001 83.890001) (width 0.25) (layer F.Cu) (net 6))
 (segment (start 133.89 85.82) (end 135.819999 83.890001) (width 0.25) (layer F.Cu) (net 6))
 (segment (start 132.08 85.82) (end 133.89 85.82) (width 0.25) (layer F.Cu) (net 6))
 (segment (start 133.675002 86.82) (end 132.08 86.82) (width 0.25) (layer F.Cu) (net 7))
 (segment (start 135.335001 85.160001) (end 133.675002 86.82) (width 0.25) (layer F.Cu) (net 7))
 (segment (start 136.585001 85.160001) (end 135.335001 85.160001) (width 0.25) (layer F.Cu) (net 7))
 (segment (start 135.335001 86.430001) (end 134.135002 87.63) (width 0.25) (layer F.Cu) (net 8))
 (segment (start 136.585001 86.430001) (end 135.335001 86.430001) (width 0.25) (layer F.Cu) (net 8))
 (segment (start 132.27 87.63) (end 132.08 87.82) (width 0.25) (layer F.Cu) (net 8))
 (segment (start 134.135002 87.63) (end 132.27 87.63) (width 0.25) (layer F.Cu) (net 8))
 (segment (start 133.581412 88.82) (end 132.08 88.82) (width 0.25) (layer F.Cu) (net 9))
 (segment (start 134.701411 87.700001) (end 133.581412 88.82) (width 0.25) (layer F.Cu) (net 9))
 (segment (start 136.585001 87.700001) (end 134.701411 87.700001) (width 0.25) (layer F.Cu) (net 9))
 (segment (start 133.217822 89.82) (end 132.08 89.82) (width 0.25) (layer F.Cu) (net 10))
 (segment (start 134.067821 88.970001) (end 133.217822 89.82) (width 0.25) (layer F.Cu) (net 10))
 (segment (start 136.585001 88.970001) (end 134.067821 88.970001) (width 0.25) (layer F.Cu) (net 10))
 (segment (start 132.854232 90.82) (end 132.08 90.82) (width 0.25) (layer F.Cu) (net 11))
 (segment (start 133.434231 90.240001) (end 132.854232 90.82) (width 0.25) (layer F.Cu) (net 11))
 (segment (start 136.585001 90.240001) (end 133.434231 90.240001) (width 0.25) (layer F.Cu) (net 11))
 (segment (start 132.190002 91.82) (end 132.08 91.82) (width 0.25) (layer F.Cu) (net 12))
 (segment (start 132.500001 91.510001) (end 132.190002 91.82) (width 0.25) (layer F.Cu) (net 12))
 (segment (start 136.585001 91.510001) (end 132.500001 91.510001) (width 0.25) (layer F.Cu) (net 12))
 (via (at 139.7 92.71) (size 0.8) (drill 0.4) (layers F.Cu B.Cu) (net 13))
 (segment (start 139.629999 92.780001) (end 139.7 92.71) (width 0.25) (layer F.Cu) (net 13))
 (segment (start 136.585001 92.780001) (end 139.629999 92.780001) (width 0.25) (layer F.Cu) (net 13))
 (segment (start 140.97 93.98) (end 168.91 93.98) (width 0.25) (layer B.Cu) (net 13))
 (segment (start 139.7 92.71) (end 140.97 93.98) (width 0.25) (layer B.Cu) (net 13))
 (via (at 140.97 91.44) (size 0.8) (drill 0.4) (layers F.Cu B.Cu) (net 15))
 (segment (start 168.91 91.44) (end 140.97 91.44) (width 0.25) (layer B.Cu) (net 15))
 (segment (start 140.97 94.720002) (end 140.640001 95.050001) (width 0.25) (layer F.Cu) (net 15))
 (segment (start 140.97 91.44) (end 140.97 94.720002) (width 0.25) (layer F.Cu) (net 15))
 (via (at 149.722349 97.652349) (size 0.8) (drill 0.4) (layers F.Cu B.Cu) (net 22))
 (segment (start 152.494999 100.424999) (end 149.722349 97.652349) (width 0.25) (layer B.Cu) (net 22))
 (segment (start 170.274999 100.424999) (end 152.494999 100.424999) (width 0.25) (layer B.Cu) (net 22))
 (segment (start 171.45 101.6) (end 170.274999 100.424999) (width 0.25) (layer B.Cu) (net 22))
 (segment (start 149.722349 95.242349) (end 149.530001 95.050001) (width 0.25) (layer F.Cu) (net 22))
 (segment (start 149.722349 97.652349) (end 149.722349 95.242349) (width 0.25) (layer F.Cu) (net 22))
 (segment (start 153.585001 94.300003) (end 153.585001 94.050001) (width 0.25) (layer F.Cu) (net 24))
 (segment (start 153.585001 94.815003) (end 153.585001 94.050001) (width 0.25) (layer F.Cu) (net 24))
 (segment (start 148.835003 99.565001) (end 153.585001 94.815003) (width 0.25) (layer F.Cu) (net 24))
 (segment (start 145.477501 99.565001) (end 148.835003 99.565001) (width 0.25) (layer F.Cu) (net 24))
 (segment (start 158.820001 91.510001) (end 153.585001 91.510001) (width 0.25) (layer F.Cu) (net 26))
 (segment (start 168.91 101.6) (end 158.820001 91.510001) (width 0.25) (layer F.Cu) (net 26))
 (via (at 156.21 87.63) (size 0.8) (drill 0.4) (layers F.Cu B.Cu) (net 29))
 (segment (start 153.655002 87.63) (end 153.585001 87.700001) (width 0.25) (layer F.Cu) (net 29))
 (segment (start 156.139999 87.700001) (end 156.21 87.63) (width 0.25) (layer F.Cu) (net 29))
 (segment (start 153.585001 87.700001) (end 156.139999 87.700001) (width 0.25) (layer F.Cu) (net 29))
 (segment (start 170.274999 87.724999) (end 156.304999 87.724999) (width 0.25) (layer B.Cu) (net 29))
 (segment (start 156.304999 87.724999) (end 156.21 87.63) (width 0.25) (layer B.Cu) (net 29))
 (segment (start 171.45 88.9) (end 170.274999 87.724999) (width 0.25) (layer B.Cu) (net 29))
 (segment (start 166.440001 86.430001) (end 153.585001 86.430001) (width 0.25) (layer F.Cu) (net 30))
 (segment (start 168.91 88.9) (end 166.440001 86.430001) (width 0.25) (layer F.Cu) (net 30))
 (via (at 160.02 88.9) (size 0.8) (drill 0.4) (layers F.Cu B.Cu) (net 32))
 (segment (start 160.02 89.369002) (end 160.02 88.9) (width 0.25) (layer F.Cu) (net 32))
 (segment (start 168.345999 97.695001) (end 160.02 89.369002) (width 0.25) (layer F.Cu) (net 32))
 (segment (start 170.085001 97.695001) (end 168.345999 97.695001) (width 0.25) (layer F.Cu) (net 32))
 (segment (start 171.45 99.06) (end 170.085001 97.695001) (width 0.25) (layer F.Cu) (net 32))
 (segment (start 160.02 88.9) (end 151.13 88.9) (width 0.25) (layer B.Cu) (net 32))
 (segment (start 152.335001 83.890001) (end 151.13 85.095002) (width 0.25) (layer F.Cu) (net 32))
 (segment (start 153.585001 83.890001) (end 152.335001 83.890001) (width 0.25) (layer F.Cu) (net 32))
 (segment (start 151.13 85.095002) (end 151.13 88.9) (width 0.25) (layer F.Cu) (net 32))
 (segment (start 151.13 88.9) (end 151.13 88.9) (width 0.25) (layer F.Cu) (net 32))
 (via (at 151.13 88.9) (size 0.8) (drill 0.4) (layers F.Cu B.Cu) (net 32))
 (segment (start 154.236409 82.620001) (end 153.585001 82.620001) (width 0.25) (layer F.Cu) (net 33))
 (segment (start 155.38641 81.47) (end 154.236409 82.620001) (width 0.25) (layer F.Cu) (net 33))
 (segment (start 171.45 81.47) (end 155.38641 81.47) (width 0.25) (layer F.Cu) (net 33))
 (segment (start 154.869999 81.350001) (end 153.585001 81.350001) (width 0.25) (layer F.Cu) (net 34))
 (segment (start 155.75 80.47) (end 154.869999 81.350001) (width 0.25) (layer F.Cu) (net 34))
 (segment (start 171.45 80.47) (end 155.75 80.47) (width 0.25) (layer F.Cu) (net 34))
 (via (at 158.75 90.17) (size 0.8) (drill 0.4) (layers F.Cu B.Cu) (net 35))
 (segment (start 167.64 99.06) (end 158.75 90.17) (width 0.25) (layer F.Cu) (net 35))
 (segment (start 168.91 99.06) (end 167.64 99.06) (width 0.25) (layer F.Cu) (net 35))
 (via (at 149.86 90.17) (size 0.8) (drill 0.4) (layers F.Cu B.Cu) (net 35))
 (segment (start 158.75 90.17) (end 149.86 90.17) (width 0.25) (layer B.Cu) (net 35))
 (segment (start 152.335001 80.080001) (end 153.585001 80.080001) (width 0.25) (layer F.Cu) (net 35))
 (segment (start 149.86 82.555002) (end 152.335001 80.080001) (width 0.25) (layer F.Cu) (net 35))
 (segment (start 149.86 90.17) (end 149.86 82.555002) (width 0.25) (layer F.Cu) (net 35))
 (segment (start 170.274999 90.264999) (end 170.274999 85.184999) (width 0.25) (layer F.Cu) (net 36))
 (segment (start 171.45 91.44) (end 170.274999 90.264999) (width 0.25) (layer F.Cu) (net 36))
 (via (at 161.29 82.55) (size 0.8) (drill 0.4) (layers F.Cu B.Cu) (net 36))
 (segment (start 167.64 82.55) (end 161.29 82.55) (width 0.25) (layer F.Cu) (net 36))
 (segment (start 170.274999 85.184999) (end 167.64 82.55) (width 0.25) (layer F.Cu) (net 36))
 (via (at 161.29 78.74) (size 0.8) (drill 0.4) (layers F.Cu B.Cu) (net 36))
 (segment (start 161.29 82.55) (end 161.29 78.74) (width 0.25) (layer B.Cu) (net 36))
 (segment (start 153.655002 78.74) (end 153.585001 78.810001) (width 0.25) (layer F.Cu) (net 36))
 (segment (start 161.29 78.74) (end 153.655002 78.74) (width 0.25) (layer F.Cu) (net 36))
 (segment (start 138.974999 107.028001) (end 138.974999 106.135001) (width 0.25) (layer B.Cu) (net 41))
 (segment (start 139.351999 107.405001) (end 138.974999 107.028001) (width 0.25) (layer B.Cu) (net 41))
 (via (at 143.51 101.6) (size 0.8) (drill 0.4) (layers F.Cu B.Cu) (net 41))
 (segment (start 141.040249 107.405001) (end 139.351999 107.405001) (width 0.25) (layer B.Cu) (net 41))
 (segment (start 138.974999 106.135001) (end 143.51 101.6) (width 0.25) (layer B.Cu) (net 41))
 (segment (start 143.51 99.707502) (end 143.652501 99.565001) (width 0.25) (layer F.Cu) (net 41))
 (segment (start 143.51 101.6) (end 143.51 99.707502) (width 0.25) (layer F.Cu) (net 41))
 (segment (start 143.51 109.874752) (end 143.51 110.49) (width 0.25) (layer B.Cu) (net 41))
 (segment (start 141.040249 107.405001) (end 143.51 109.874752) (width 0.25) (layer B.Cu) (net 41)))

